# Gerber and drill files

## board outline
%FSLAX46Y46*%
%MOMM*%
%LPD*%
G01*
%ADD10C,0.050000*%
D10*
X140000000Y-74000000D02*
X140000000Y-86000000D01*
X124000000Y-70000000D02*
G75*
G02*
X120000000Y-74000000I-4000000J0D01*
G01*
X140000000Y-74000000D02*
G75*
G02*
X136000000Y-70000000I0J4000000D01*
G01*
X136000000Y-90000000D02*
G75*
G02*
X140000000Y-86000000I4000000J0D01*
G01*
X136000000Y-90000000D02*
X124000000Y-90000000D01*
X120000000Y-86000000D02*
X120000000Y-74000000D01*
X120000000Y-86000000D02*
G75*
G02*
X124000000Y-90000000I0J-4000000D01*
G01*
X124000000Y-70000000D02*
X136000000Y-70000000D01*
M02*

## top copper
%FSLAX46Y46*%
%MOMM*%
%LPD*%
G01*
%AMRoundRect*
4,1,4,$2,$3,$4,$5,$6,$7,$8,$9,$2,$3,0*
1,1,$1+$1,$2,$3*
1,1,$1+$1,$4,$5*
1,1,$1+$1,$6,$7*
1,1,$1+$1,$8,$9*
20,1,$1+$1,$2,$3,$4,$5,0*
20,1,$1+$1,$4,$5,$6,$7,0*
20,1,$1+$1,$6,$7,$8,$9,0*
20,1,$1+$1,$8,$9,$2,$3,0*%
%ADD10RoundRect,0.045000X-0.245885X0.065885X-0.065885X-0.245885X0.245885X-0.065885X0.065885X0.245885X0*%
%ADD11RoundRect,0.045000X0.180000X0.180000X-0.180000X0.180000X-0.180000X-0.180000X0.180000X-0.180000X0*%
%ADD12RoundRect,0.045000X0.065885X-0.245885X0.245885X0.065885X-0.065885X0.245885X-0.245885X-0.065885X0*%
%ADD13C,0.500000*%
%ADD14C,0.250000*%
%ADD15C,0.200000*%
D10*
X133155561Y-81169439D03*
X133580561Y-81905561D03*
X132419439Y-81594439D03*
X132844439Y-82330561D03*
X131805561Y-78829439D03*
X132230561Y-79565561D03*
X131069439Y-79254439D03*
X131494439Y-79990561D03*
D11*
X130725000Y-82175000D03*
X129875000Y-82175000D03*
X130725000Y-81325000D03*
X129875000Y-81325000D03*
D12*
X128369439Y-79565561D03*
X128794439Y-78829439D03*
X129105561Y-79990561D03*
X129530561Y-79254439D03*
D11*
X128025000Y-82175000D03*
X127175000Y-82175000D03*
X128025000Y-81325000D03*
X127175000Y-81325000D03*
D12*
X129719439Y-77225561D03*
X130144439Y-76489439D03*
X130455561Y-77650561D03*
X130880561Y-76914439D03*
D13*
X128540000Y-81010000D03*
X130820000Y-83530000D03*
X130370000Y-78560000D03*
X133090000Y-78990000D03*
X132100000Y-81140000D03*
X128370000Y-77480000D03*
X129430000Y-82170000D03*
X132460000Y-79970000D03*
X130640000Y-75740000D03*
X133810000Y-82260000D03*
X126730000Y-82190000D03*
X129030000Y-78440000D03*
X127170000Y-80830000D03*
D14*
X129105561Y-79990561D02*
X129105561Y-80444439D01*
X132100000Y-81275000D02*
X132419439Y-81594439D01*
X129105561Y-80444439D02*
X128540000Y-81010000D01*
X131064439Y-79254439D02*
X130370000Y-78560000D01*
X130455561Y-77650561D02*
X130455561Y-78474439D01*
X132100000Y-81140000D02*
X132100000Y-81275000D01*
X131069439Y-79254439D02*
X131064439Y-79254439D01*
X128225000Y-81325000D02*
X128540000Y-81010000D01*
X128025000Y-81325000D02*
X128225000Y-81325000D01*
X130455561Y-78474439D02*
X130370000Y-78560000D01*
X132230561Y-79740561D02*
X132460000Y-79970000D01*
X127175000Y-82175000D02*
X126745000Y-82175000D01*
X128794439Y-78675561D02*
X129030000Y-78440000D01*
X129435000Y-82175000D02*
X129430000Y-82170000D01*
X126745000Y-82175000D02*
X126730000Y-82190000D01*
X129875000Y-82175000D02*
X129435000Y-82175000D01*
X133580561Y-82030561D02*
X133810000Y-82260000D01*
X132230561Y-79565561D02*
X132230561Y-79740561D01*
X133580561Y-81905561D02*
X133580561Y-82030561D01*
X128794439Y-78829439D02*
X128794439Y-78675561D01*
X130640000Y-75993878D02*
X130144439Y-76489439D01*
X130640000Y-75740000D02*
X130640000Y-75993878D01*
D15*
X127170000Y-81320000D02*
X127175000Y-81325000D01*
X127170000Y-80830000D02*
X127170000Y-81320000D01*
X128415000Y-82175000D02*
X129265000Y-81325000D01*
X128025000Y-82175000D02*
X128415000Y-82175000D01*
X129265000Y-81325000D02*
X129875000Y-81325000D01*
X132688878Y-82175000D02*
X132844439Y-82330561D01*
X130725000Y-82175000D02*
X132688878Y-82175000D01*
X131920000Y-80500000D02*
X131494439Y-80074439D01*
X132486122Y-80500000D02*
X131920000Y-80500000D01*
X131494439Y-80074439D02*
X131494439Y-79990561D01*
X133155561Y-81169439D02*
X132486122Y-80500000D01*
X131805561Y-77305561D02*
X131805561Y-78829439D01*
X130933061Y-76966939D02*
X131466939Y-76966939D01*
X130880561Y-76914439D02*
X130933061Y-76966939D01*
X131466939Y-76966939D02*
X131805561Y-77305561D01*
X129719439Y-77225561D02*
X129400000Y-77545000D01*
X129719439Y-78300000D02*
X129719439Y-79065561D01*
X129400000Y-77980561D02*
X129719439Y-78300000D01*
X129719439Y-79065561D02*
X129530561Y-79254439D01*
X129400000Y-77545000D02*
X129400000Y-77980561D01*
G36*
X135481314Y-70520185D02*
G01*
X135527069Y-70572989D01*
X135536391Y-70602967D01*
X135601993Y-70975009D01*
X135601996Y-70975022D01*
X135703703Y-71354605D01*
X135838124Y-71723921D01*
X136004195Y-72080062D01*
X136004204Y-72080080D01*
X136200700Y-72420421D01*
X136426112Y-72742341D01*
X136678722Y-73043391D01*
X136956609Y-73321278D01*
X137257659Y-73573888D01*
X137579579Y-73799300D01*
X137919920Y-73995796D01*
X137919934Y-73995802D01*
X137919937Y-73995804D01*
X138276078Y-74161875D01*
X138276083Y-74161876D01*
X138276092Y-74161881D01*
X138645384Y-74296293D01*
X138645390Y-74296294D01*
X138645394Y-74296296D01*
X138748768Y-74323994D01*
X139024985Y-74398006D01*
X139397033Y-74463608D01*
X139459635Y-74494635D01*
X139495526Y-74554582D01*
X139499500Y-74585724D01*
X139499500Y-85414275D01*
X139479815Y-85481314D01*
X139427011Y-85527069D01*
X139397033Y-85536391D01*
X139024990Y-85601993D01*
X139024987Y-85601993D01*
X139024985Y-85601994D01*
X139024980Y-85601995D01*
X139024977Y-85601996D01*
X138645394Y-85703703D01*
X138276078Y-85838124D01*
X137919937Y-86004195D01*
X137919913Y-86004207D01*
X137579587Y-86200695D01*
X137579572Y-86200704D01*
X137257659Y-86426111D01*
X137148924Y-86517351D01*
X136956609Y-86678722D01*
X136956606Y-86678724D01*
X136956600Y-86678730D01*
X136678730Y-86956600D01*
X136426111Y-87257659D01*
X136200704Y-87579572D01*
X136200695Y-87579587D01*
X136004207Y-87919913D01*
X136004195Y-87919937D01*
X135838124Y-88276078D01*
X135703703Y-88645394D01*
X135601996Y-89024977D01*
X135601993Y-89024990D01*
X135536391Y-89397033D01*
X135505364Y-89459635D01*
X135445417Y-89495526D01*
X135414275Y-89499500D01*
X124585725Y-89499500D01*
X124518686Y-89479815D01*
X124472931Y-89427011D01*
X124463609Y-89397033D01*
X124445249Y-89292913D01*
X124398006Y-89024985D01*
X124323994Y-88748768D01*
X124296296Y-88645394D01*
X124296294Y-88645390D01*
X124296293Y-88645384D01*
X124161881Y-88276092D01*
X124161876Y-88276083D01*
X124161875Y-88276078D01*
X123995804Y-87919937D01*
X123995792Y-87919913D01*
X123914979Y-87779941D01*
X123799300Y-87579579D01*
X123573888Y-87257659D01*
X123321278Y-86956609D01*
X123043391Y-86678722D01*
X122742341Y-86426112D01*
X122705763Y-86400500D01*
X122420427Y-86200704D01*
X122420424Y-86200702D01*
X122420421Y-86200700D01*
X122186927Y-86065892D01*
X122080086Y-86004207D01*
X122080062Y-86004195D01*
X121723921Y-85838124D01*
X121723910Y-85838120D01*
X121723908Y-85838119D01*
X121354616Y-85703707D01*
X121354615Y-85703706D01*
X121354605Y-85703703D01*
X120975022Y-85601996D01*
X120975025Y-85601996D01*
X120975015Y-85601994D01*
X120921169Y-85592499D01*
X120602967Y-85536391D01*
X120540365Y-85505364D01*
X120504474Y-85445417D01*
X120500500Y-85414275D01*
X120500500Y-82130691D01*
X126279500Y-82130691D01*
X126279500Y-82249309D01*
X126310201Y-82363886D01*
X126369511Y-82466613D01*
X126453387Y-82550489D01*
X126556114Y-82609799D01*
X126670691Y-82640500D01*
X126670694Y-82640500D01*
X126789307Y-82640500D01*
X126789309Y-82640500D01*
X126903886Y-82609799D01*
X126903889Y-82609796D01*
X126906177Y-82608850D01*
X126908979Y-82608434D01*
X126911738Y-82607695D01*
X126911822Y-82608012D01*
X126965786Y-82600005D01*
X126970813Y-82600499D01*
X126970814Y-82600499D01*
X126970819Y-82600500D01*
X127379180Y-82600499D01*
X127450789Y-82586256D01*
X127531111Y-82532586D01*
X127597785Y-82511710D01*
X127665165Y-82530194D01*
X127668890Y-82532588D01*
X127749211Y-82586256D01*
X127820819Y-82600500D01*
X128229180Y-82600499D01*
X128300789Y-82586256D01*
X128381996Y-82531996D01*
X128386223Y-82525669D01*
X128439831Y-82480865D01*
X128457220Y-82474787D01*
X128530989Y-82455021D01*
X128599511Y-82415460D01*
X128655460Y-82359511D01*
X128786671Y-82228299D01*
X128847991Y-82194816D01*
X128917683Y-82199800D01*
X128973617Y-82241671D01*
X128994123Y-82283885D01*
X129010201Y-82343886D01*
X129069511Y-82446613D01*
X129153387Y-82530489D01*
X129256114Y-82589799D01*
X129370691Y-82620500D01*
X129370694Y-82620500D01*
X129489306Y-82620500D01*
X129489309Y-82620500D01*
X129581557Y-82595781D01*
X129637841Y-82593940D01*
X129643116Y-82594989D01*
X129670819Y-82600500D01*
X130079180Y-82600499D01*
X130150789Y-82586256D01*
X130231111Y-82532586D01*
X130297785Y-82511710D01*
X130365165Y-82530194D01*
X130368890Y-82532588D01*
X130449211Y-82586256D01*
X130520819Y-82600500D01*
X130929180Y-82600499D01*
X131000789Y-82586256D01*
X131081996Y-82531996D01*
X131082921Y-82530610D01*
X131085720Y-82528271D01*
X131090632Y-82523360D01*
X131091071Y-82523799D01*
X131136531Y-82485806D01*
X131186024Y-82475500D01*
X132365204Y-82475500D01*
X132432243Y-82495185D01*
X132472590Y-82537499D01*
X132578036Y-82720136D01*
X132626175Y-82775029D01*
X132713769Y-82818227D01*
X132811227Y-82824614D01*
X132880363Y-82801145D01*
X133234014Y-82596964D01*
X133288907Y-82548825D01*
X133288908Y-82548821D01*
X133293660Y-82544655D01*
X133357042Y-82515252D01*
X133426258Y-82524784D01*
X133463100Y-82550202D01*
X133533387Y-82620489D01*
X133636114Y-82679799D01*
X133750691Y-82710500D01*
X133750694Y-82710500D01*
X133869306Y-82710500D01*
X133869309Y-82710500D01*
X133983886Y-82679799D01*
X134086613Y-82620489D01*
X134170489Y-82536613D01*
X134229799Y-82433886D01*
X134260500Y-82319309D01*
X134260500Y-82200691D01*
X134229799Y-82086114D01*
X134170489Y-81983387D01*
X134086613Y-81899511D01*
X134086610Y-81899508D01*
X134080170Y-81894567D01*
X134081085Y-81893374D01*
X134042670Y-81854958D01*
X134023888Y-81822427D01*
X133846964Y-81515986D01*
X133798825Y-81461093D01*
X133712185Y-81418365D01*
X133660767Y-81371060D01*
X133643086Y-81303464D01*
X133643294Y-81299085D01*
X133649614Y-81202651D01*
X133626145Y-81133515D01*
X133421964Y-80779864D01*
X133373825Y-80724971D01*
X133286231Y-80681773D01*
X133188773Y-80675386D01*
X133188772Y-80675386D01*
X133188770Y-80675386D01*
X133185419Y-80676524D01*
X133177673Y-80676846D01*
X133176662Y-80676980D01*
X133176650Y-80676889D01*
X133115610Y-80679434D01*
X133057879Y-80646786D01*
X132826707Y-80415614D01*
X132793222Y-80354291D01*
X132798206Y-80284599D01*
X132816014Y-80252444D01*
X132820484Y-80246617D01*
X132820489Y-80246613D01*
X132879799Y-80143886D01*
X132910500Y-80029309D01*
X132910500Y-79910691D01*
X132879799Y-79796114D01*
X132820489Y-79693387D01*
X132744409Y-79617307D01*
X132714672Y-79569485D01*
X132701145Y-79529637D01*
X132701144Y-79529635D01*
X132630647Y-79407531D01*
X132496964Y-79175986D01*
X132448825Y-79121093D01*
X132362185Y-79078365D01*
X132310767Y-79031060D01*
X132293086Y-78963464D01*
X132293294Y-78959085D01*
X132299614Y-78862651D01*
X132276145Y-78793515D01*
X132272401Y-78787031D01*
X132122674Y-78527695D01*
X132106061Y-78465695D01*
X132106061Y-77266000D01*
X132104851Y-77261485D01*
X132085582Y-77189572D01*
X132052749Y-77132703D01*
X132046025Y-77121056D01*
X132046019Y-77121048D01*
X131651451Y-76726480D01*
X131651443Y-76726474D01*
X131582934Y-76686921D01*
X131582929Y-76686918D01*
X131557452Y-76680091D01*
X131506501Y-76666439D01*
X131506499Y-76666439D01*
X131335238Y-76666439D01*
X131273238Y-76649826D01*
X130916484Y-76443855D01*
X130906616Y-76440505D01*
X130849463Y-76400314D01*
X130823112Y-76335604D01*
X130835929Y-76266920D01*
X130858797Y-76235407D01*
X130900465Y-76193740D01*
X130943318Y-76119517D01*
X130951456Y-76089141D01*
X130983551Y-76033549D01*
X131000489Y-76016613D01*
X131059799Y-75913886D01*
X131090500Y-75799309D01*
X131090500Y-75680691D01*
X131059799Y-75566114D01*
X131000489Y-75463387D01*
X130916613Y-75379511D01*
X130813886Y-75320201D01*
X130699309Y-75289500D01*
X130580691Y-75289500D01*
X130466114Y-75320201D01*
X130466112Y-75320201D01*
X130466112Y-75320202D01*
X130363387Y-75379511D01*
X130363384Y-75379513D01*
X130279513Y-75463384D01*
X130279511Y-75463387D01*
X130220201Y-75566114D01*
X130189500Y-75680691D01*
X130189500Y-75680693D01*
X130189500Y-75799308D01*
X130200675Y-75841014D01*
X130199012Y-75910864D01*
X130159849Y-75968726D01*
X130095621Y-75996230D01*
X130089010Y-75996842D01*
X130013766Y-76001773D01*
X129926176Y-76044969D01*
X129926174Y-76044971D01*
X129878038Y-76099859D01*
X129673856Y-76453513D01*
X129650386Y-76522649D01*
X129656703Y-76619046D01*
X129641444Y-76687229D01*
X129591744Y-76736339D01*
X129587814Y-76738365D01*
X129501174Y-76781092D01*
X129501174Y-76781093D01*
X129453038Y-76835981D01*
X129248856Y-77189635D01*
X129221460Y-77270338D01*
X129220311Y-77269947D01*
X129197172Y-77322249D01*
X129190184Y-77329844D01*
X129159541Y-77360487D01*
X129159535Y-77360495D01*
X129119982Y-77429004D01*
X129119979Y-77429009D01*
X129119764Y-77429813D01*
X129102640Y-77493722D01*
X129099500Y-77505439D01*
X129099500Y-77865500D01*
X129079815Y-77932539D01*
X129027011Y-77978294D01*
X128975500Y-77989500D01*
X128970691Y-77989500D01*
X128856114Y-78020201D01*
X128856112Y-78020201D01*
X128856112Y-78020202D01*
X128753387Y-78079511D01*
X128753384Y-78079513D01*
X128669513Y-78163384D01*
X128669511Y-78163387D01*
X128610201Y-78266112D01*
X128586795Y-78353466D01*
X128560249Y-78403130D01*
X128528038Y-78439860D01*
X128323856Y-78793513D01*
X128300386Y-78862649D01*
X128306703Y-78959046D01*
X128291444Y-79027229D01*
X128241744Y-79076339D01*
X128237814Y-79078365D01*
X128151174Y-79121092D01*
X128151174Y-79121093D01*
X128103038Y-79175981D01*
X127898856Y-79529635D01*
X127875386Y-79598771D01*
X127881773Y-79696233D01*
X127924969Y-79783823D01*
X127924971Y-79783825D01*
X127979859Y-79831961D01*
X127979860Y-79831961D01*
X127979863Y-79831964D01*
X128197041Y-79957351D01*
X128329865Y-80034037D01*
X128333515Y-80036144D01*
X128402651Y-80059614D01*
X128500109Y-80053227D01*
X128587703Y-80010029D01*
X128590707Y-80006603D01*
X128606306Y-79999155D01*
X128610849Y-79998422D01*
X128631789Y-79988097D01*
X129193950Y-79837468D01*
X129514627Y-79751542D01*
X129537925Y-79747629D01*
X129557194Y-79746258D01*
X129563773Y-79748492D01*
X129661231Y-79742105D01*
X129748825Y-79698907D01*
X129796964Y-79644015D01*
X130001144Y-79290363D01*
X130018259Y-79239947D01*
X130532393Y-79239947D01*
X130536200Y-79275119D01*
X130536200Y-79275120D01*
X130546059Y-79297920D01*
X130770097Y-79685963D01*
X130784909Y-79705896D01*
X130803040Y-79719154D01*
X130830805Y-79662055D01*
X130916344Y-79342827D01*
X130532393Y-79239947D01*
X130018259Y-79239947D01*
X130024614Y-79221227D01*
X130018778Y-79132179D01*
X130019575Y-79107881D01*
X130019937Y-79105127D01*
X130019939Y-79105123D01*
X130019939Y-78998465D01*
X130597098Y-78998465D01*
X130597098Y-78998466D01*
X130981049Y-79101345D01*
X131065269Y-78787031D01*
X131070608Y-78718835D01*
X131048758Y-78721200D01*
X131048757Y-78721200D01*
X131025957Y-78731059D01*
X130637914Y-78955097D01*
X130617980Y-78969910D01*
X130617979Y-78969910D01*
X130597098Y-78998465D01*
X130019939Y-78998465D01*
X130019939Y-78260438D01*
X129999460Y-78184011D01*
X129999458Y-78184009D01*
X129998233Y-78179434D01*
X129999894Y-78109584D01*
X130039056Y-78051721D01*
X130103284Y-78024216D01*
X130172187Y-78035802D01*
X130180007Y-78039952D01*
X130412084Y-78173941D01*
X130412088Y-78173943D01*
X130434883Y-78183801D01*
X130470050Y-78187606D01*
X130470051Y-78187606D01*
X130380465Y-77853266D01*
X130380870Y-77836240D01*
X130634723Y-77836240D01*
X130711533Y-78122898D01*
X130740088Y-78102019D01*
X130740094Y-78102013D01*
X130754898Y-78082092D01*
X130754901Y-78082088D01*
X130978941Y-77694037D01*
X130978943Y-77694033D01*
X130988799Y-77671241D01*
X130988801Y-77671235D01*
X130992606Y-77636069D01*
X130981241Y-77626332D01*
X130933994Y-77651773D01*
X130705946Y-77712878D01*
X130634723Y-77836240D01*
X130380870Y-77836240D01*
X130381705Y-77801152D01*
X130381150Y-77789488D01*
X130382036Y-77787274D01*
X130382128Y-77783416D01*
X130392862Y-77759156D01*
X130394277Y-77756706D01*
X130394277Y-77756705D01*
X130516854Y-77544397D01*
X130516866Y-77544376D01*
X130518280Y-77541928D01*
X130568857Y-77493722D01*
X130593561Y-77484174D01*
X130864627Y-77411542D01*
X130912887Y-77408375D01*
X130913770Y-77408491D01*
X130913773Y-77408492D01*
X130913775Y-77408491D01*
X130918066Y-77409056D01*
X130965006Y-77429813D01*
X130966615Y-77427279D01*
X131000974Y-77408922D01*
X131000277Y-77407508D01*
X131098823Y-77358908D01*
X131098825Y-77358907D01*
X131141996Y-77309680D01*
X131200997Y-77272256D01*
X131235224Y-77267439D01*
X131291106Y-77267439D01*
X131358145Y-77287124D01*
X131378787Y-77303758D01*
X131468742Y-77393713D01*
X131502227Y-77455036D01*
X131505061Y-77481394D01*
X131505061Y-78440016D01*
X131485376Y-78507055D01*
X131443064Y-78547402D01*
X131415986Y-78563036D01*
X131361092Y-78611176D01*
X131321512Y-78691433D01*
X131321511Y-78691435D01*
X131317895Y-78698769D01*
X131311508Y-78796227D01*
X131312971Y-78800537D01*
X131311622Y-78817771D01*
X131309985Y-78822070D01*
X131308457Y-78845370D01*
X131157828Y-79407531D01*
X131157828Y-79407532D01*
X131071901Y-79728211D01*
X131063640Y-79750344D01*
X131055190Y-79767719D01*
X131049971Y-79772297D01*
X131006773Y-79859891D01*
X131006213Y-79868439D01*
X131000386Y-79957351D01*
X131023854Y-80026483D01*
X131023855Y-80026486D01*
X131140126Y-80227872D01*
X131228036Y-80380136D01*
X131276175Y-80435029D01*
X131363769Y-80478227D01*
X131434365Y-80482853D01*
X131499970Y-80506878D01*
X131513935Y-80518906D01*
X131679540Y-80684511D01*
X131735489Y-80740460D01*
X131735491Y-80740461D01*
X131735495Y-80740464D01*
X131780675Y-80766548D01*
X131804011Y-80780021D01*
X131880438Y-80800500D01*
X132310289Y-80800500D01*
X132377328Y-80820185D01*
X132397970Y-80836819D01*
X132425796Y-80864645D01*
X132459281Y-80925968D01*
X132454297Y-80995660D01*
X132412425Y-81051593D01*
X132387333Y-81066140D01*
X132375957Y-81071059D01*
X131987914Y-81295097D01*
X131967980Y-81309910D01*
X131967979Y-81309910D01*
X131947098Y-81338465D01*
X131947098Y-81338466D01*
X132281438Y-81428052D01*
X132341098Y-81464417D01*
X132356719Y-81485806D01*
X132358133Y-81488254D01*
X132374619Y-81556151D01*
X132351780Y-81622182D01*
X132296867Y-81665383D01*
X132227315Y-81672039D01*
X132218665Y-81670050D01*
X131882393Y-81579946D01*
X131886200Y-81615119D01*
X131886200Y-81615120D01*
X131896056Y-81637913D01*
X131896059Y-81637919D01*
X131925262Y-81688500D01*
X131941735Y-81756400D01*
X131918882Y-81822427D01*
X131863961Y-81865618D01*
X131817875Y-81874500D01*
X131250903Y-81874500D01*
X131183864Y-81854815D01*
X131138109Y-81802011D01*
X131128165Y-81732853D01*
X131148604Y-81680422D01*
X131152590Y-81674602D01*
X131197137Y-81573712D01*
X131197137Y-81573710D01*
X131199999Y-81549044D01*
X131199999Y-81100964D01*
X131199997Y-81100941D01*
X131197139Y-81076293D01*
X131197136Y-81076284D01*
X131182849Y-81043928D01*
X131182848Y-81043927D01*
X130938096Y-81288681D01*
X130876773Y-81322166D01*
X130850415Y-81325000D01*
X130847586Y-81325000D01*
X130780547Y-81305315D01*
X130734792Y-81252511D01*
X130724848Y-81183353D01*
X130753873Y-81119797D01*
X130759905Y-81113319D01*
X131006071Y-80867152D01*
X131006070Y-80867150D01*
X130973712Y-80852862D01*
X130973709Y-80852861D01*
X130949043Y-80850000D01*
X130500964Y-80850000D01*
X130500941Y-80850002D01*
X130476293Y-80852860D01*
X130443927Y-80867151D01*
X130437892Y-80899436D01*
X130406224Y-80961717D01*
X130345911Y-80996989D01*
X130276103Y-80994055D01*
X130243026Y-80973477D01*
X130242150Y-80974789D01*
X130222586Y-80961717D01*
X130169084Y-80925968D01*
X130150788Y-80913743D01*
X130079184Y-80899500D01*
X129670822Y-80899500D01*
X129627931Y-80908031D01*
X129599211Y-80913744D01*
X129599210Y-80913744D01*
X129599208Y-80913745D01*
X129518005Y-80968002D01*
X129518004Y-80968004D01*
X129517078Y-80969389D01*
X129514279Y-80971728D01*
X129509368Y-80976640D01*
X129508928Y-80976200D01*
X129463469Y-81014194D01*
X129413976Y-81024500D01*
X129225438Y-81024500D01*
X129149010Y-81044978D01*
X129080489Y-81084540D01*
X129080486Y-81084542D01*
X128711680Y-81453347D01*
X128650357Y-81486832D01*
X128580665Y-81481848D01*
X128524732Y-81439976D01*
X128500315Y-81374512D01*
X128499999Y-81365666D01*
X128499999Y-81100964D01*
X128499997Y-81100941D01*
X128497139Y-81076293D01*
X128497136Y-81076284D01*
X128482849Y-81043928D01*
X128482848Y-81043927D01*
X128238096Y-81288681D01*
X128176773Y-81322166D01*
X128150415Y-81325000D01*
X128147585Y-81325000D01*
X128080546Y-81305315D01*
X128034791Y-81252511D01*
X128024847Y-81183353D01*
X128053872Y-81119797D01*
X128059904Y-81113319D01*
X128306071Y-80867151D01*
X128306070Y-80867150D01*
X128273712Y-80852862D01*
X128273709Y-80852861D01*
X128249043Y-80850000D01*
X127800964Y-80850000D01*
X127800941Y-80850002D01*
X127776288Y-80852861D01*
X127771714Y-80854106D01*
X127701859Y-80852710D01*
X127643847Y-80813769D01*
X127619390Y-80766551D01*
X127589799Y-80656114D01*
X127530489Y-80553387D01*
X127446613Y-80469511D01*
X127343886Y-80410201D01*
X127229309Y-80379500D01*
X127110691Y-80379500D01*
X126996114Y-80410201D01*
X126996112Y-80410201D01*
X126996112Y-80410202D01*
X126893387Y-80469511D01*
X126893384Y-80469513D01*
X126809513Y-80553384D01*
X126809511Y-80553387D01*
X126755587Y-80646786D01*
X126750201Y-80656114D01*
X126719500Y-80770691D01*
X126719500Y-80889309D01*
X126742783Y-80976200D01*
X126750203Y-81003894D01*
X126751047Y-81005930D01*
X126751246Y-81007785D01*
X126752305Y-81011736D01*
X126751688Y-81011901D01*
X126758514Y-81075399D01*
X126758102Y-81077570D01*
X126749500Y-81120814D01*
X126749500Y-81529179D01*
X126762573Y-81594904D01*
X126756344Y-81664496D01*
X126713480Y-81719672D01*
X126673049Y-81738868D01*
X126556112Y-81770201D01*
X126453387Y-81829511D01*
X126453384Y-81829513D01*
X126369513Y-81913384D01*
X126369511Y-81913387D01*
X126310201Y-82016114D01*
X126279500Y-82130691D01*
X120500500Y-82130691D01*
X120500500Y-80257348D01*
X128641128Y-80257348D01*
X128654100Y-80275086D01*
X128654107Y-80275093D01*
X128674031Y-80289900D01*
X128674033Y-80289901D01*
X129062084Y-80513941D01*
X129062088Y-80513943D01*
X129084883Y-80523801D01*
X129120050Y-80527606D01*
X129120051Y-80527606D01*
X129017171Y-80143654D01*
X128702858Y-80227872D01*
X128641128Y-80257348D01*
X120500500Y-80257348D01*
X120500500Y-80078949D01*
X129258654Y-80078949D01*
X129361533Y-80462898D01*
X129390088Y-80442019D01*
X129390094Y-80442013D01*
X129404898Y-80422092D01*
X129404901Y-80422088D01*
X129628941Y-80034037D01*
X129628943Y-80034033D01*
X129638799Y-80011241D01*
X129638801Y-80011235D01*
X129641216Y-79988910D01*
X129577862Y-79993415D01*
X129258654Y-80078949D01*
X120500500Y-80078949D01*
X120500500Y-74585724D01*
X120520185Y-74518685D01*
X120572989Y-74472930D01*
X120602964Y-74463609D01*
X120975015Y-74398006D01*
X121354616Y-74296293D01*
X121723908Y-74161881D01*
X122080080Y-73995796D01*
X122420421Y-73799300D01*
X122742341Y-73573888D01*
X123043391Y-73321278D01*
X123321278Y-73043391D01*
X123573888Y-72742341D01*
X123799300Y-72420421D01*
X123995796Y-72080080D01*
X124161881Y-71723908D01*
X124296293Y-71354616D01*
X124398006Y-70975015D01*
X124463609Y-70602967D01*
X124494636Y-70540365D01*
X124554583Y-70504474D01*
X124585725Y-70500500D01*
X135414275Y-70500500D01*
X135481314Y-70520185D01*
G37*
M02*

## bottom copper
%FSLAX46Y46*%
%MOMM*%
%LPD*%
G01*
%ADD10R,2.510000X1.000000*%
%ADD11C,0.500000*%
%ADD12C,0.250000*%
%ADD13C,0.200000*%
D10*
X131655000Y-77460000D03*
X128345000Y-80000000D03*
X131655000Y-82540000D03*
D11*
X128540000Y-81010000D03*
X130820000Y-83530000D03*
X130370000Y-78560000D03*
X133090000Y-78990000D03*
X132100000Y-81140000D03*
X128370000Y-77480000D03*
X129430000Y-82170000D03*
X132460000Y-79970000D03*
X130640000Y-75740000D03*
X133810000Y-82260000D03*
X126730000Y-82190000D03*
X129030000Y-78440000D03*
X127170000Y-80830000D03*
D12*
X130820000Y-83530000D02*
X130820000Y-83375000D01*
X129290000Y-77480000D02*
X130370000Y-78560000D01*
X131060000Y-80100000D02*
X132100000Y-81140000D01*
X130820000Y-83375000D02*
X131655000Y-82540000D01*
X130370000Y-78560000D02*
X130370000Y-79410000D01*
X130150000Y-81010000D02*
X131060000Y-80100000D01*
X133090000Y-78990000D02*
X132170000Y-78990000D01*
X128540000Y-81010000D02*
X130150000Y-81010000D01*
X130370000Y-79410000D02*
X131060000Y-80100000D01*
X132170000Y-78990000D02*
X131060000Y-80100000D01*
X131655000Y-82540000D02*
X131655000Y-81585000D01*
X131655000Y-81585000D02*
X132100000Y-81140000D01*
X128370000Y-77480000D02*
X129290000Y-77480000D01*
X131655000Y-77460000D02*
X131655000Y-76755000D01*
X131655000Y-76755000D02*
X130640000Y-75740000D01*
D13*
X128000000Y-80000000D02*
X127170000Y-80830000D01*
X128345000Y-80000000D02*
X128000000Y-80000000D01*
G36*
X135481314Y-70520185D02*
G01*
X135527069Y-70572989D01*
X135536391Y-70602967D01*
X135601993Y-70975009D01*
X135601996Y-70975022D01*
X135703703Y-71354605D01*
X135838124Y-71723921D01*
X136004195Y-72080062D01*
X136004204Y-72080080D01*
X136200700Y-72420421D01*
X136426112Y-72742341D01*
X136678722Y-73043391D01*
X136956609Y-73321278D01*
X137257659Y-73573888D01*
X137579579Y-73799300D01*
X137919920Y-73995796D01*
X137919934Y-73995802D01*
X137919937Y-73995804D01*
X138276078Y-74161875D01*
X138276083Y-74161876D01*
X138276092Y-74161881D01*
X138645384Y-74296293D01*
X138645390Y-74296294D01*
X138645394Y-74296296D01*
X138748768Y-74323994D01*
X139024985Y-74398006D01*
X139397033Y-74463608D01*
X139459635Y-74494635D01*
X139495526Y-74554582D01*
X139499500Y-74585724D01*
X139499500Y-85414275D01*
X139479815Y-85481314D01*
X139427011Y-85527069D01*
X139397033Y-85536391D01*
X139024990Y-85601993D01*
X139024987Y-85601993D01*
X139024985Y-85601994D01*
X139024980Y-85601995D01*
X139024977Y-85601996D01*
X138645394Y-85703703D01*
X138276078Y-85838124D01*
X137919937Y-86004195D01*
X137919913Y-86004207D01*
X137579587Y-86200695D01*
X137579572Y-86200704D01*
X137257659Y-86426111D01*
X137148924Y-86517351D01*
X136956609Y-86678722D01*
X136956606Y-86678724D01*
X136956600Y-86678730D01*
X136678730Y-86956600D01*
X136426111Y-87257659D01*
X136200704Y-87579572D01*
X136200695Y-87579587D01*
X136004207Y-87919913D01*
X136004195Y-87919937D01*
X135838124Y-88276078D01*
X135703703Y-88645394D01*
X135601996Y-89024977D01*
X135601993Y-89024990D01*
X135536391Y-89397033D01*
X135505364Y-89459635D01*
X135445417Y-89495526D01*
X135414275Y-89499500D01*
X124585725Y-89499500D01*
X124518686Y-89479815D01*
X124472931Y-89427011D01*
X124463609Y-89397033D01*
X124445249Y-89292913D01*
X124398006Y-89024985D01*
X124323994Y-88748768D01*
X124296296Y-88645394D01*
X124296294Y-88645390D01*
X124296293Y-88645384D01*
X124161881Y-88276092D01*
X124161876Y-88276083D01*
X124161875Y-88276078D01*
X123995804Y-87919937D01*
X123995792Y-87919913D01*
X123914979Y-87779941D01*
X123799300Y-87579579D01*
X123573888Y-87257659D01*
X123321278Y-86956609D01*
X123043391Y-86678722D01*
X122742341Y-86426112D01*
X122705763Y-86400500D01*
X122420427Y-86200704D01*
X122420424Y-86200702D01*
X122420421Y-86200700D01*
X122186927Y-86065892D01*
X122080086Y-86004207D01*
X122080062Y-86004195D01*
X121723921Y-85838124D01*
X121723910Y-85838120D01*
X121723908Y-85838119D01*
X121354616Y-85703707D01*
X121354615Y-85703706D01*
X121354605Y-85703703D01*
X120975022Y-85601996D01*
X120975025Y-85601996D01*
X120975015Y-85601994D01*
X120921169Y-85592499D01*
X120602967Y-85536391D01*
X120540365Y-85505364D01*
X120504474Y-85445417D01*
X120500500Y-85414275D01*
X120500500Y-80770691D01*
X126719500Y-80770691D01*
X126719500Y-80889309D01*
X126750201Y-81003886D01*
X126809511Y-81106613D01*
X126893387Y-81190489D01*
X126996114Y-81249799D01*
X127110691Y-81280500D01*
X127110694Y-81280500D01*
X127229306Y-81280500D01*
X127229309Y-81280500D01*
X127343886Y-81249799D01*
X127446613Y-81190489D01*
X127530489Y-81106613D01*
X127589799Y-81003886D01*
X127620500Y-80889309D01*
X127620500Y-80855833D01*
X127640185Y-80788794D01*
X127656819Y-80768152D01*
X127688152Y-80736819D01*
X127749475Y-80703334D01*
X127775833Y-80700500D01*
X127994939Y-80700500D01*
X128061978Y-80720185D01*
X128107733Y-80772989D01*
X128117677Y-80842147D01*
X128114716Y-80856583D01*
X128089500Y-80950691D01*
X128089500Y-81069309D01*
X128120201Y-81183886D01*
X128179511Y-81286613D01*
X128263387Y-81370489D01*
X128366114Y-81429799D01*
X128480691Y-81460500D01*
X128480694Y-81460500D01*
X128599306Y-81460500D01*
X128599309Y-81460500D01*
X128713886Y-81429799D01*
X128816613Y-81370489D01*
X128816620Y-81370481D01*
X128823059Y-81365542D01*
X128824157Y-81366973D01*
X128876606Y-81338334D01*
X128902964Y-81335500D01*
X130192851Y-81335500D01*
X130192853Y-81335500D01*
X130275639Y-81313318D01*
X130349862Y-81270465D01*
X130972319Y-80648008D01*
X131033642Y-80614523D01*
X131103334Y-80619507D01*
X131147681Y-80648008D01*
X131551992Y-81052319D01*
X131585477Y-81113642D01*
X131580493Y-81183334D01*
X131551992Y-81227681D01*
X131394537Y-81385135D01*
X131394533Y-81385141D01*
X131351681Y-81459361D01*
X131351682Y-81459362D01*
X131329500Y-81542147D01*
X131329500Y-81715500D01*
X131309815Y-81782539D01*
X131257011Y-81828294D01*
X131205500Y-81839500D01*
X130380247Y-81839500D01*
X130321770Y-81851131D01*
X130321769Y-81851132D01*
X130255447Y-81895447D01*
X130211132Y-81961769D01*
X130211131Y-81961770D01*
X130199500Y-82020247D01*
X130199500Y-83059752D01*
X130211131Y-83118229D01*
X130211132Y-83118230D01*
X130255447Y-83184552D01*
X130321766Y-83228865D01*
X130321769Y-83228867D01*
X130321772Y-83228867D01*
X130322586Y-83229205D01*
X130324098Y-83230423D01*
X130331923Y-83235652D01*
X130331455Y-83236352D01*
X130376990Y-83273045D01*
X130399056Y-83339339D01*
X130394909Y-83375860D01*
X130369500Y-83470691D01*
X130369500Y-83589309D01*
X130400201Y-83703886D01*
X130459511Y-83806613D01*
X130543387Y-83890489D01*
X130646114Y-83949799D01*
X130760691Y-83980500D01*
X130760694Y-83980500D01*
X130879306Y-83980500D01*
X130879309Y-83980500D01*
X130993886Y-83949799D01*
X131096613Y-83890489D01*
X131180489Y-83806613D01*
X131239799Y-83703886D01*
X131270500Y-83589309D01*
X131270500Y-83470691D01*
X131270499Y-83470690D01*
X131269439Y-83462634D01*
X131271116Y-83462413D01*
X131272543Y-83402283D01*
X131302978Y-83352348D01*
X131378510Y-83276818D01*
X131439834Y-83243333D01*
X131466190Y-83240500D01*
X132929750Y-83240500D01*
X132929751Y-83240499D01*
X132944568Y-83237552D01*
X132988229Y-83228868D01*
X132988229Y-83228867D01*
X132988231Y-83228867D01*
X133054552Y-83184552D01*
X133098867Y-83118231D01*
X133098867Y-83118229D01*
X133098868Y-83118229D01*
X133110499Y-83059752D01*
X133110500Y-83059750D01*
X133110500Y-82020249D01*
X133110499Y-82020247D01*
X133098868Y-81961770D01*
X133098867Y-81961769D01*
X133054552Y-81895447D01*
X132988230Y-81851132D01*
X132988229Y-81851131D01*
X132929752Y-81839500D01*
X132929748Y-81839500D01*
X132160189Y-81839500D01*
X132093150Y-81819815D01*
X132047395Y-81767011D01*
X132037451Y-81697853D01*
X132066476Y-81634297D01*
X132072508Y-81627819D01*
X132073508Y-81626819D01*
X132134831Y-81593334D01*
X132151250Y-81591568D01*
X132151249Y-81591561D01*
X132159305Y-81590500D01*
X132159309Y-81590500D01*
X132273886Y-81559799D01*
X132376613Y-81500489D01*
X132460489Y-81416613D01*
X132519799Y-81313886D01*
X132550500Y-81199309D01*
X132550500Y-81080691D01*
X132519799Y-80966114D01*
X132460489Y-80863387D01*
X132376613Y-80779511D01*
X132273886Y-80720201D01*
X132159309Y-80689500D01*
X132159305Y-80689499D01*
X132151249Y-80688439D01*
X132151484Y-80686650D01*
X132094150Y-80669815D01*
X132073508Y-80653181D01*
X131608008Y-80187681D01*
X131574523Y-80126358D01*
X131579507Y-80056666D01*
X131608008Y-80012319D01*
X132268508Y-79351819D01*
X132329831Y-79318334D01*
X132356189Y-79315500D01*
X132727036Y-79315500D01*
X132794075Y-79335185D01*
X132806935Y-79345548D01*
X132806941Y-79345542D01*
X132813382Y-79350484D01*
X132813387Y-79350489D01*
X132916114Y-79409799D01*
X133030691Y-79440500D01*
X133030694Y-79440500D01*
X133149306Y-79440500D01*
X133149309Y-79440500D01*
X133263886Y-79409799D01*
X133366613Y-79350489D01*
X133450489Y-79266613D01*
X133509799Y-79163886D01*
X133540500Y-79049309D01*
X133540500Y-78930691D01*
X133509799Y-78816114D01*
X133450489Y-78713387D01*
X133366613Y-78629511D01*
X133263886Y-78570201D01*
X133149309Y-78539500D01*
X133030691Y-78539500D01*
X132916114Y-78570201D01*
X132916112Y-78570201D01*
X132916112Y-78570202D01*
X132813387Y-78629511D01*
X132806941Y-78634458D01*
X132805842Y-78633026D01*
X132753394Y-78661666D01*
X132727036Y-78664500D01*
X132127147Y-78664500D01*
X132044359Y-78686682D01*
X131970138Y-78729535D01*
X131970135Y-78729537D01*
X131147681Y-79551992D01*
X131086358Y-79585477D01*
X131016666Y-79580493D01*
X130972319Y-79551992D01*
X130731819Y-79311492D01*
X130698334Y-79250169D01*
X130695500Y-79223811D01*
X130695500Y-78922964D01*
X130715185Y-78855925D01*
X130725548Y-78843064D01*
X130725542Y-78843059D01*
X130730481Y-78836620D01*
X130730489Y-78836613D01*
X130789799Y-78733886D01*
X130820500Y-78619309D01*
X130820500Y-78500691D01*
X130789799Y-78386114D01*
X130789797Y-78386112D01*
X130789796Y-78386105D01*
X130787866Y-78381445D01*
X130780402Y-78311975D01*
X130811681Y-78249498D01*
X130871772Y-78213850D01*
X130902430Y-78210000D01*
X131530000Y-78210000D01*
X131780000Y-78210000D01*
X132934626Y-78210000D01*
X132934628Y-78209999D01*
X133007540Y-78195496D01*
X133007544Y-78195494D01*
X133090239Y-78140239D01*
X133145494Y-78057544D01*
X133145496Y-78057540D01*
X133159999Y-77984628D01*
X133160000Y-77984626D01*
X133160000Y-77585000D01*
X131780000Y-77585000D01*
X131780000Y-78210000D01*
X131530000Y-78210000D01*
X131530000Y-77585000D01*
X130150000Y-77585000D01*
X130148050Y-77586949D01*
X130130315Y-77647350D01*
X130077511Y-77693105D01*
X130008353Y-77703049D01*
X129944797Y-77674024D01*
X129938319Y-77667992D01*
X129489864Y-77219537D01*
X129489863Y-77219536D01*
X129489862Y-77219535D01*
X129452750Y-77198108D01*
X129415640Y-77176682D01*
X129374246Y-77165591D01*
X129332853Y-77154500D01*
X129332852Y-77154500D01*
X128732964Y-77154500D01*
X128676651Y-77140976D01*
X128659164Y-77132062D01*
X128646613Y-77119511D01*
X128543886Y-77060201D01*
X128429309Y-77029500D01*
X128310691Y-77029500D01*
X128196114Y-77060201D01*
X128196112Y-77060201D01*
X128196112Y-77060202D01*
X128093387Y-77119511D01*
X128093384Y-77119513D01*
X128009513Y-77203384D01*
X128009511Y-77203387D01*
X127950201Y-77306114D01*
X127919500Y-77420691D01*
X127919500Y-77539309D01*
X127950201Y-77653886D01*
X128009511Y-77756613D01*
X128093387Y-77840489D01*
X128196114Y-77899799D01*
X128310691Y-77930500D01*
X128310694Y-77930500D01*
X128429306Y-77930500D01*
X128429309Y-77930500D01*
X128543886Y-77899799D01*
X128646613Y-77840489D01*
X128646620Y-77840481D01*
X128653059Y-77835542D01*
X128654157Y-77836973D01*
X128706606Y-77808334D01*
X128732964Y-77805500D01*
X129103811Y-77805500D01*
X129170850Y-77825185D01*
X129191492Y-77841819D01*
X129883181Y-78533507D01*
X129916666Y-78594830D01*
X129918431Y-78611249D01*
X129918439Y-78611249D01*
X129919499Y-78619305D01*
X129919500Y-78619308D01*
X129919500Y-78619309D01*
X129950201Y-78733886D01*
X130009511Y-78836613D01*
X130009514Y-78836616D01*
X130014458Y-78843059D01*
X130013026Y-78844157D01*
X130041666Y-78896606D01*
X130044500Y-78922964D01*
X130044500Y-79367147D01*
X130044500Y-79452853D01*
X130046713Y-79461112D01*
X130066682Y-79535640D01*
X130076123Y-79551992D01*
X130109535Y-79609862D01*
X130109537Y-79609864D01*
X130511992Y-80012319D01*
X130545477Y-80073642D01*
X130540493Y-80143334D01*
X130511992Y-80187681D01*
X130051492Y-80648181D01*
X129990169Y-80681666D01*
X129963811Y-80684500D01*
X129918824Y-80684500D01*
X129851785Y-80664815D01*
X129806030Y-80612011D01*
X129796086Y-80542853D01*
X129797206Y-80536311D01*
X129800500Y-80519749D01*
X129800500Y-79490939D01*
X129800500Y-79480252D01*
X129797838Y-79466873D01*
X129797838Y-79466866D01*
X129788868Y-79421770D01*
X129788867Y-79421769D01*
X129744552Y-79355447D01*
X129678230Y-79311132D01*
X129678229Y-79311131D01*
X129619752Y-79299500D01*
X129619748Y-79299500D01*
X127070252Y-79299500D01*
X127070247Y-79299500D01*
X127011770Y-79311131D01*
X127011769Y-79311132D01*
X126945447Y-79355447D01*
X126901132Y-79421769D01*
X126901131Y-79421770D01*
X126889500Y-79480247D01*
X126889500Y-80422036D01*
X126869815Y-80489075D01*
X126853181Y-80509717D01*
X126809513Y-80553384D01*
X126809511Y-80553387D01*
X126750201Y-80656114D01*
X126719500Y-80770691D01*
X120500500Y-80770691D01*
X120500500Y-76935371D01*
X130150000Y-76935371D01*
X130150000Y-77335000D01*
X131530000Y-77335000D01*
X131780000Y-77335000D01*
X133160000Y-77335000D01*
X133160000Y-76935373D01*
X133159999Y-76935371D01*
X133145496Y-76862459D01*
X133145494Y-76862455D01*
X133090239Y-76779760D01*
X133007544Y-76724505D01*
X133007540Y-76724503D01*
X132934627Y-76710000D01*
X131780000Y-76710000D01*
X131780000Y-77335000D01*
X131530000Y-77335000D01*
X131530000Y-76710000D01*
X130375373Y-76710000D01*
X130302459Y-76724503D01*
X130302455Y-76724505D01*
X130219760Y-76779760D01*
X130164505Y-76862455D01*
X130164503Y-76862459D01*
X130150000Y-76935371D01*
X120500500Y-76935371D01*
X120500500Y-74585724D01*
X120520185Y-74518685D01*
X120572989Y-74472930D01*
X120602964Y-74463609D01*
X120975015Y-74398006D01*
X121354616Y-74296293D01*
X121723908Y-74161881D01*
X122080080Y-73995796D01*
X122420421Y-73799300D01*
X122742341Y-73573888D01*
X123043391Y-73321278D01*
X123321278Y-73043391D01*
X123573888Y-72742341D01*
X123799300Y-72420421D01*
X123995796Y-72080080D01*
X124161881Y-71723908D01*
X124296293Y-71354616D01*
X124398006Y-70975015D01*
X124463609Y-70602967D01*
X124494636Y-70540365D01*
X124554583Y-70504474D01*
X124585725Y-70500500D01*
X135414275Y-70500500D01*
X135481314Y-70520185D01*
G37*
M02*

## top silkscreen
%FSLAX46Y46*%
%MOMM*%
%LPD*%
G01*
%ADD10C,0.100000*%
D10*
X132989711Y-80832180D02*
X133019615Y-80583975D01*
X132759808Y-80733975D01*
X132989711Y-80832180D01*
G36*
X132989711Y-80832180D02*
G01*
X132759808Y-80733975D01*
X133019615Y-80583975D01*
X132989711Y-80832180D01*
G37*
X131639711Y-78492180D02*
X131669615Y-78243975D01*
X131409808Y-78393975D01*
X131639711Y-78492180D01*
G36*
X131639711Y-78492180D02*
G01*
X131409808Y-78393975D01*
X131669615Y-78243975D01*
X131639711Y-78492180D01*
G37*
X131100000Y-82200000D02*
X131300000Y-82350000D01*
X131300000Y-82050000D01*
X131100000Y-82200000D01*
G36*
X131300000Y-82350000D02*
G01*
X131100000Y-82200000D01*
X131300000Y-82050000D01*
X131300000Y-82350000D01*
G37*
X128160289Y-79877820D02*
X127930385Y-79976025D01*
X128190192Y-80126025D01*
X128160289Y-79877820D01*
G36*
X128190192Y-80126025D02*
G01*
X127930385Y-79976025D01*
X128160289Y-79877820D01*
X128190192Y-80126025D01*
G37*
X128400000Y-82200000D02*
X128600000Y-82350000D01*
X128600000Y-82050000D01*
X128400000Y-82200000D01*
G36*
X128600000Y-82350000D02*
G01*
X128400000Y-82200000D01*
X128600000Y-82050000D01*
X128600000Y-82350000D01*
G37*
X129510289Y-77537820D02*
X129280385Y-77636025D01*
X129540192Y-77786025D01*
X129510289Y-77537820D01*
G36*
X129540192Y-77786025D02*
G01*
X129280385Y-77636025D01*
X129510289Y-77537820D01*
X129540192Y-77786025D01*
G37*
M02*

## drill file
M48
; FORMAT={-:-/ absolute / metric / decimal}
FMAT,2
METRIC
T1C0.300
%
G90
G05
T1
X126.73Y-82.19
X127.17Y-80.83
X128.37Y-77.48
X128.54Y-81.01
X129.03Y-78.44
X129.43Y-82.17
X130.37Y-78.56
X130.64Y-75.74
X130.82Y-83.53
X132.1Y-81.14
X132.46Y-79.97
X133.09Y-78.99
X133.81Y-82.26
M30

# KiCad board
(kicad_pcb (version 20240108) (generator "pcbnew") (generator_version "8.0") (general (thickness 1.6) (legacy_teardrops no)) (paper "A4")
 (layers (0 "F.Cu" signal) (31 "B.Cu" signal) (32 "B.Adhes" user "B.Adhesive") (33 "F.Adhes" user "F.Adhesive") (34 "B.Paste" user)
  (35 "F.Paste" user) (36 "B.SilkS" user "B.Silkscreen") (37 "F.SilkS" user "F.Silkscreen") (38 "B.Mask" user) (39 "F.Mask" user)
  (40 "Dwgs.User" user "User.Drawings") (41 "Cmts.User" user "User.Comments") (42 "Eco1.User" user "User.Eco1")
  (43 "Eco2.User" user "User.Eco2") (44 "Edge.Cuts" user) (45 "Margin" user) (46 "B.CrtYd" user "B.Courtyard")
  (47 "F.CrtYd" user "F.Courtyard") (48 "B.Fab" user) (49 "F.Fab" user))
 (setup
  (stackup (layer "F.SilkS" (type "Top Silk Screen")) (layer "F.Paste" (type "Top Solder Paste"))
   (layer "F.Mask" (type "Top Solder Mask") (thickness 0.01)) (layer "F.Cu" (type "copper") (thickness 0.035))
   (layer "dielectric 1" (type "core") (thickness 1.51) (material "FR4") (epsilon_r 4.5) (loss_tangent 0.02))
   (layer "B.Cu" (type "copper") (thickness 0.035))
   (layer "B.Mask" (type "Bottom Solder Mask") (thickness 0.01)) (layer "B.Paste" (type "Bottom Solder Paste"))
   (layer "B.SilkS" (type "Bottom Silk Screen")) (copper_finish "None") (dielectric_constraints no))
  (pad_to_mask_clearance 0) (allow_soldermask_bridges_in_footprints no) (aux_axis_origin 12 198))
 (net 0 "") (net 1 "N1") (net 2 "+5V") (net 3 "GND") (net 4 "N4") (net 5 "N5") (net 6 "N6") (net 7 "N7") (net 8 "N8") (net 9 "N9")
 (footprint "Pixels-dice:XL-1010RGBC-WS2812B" (layer "F.Cu") (at 133 81.75 -60)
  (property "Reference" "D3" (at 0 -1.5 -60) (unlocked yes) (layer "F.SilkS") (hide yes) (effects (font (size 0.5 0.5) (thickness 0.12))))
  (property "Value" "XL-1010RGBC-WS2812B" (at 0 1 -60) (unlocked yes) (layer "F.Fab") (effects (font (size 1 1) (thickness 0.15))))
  (fp_poly (pts (xy -0.8 -0.449999) (xy -1 -0.6) (xy -0.999999 -0.3)) (stroke (width 0.1) (type solid)) (fill solid) (layer "F.SilkS"))
  (pad "1" smd roundrect (at -0.425 -0.425 300) (size 0.45 0.45) (layers "F.Cu" "F.Paste" "F.Mask") (roundrect_rratio 0.1) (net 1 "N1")
   (thermal_bridge_angle 45))
  (pad "2" smd roundrect (at 0.425 -0.425 300) (size 0.45 0.45) (layers "F.Cu" "F.Paste" "F.Mask") (roundrect_rratio 0.1) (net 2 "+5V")
   (thermal_bridge_angle 45))
  (pad "3" smd roundrect (at -0.425 0.425 300) (size 0.45 0.45) (layers "F.Cu" "F.Paste" "F.Mask") (roundrect_rratio 0.1) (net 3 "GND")
   (thermal_bridge_angle 45))
  (pad "4" smd roundrect (at 0.425 0.425 300) (size 0.45 0.45) (layers "F.Cu" "F.Paste" "F.Mask") (roundrect_rratio 0.1) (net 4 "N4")
   (thermal_bridge_angle 45)))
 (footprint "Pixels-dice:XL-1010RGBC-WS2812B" (layer "F.Cu") (at 131.65 79.41 -60)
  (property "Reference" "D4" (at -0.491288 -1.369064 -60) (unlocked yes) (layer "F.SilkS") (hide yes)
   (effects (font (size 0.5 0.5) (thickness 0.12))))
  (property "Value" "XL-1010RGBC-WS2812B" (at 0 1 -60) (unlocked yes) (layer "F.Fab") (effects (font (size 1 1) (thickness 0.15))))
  (fp_poly (pts (xy -0.8 -0.449999) (xy -1 -0.6) (xy -0.999999 -0.3)) (stroke (width 0.1) (type solid)) (fill solid) (layer "F.SilkS"))
  (pad "1" smd roundrect (at -0.425 -0.425 300) (size 0.45 0.45) (layers "F.Cu" "F.Paste" "F.Mask") (roundrect_rratio 0.1) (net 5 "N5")
   (thermal_bridge_angle 45))
  (pad "2" smd roundrect (at 0.425 -0.425 300) (size 0.45 0.45) (layers "F.Cu" "F.Paste" "F.Mask") (roundrect_rratio 0.1) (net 2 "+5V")
   (thermal_bridge_angle 45))
  (pad "3" smd roundrect (at -0.425 0.425 300) (size 0.45 0.45) (layers "F.Cu" "F.Paste" "F.Mask") (roundrect_rratio 0.1) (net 3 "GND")
   (thermal_bridge_angle 45))
  (pad "4" smd roundrect (at 0.425 0.425 300) (size 0.45 0.45) (layers "F.Cu" "F.Paste" "F.Mask") (roundrect_rratio 0.1) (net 1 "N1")
   (thermal_bridge_angle 45)))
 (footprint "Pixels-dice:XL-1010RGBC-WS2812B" (layer "F.Cu") (at 130.3 81.75 180)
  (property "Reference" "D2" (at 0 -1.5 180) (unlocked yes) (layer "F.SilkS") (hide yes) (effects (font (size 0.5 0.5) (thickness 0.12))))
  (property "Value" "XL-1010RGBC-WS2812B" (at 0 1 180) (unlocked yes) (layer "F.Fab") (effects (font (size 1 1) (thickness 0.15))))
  (fp_poly (pts (xy -0.8 -0.45) (xy -1 -0.6) (xy -1 -0.3)) (stroke (width 0.1) (type solid)) (fill solid) (layer "F.SilkS"))
  (pad "1" smd roundrect (at -0.425 -0.425 180) (size 0.45 0.45) (layers "F.Cu" "F.Paste" "F.Mask") (roundrect_rratio 0.1) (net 4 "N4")
   (thermal_bridge_angle 45))
  (pad "2" smd roundrect (at 0.425 -0.425 180) (size 0.45 0.45) (layers "F.Cu" "F.Paste" "F.Mask") (roundrect_rratio 0.1) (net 2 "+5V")
   (thermal_bridge_angle 45))
  (pad "3" smd roundrect (at -0.425 0.425 180) (size 0.45 0.45) (layers "F.Cu" "F.Paste" "F.Mask") (roundrect_rratio 0.1) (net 3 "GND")
   (thermal_bridge_angle 45))
  (pad "4" smd roundrect (at 0.425 0.425 180) (size 0.45 0.45) (layers "F.Cu" "F.Paste" "F.Mask") (roundrect_rratio 0.1) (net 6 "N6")
   (thermal_bridge_angle 45)))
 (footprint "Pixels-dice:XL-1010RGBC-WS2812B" (layer "F.Cu") (at 128.95 79.41 60)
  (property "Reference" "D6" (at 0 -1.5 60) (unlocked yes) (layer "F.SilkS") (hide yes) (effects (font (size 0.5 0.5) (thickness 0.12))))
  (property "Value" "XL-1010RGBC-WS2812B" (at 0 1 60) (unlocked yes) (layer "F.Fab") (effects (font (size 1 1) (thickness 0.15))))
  (fp_poly (pts (xy -0.8 -0.45) (xy -1 -0.6) (xy -1 -0.300001)) (stroke (width 0.1) (type solid)) (fill solid) (layer "F.SilkS"))
  (pad "1" smd roundrect (at -0.425 -0.425 60) (size 0.45 0.45) (layers "F.Cu" "F.Paste" "F.Mask") (roundrect_rratio 0.1) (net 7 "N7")
   (thermal_bridge_angle 45))
  (pad "2" smd roundrect (at 0.425 -0.425 60) (size 0.45 0.45) (layers "F.Cu" "F.Paste" "F.Mask") (roundrect_rratio 0.1) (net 2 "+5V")
   (thermal_bridge_angle 45))
  (pad "3" smd roundrect (at -0.425 0.425 60) (size 0.45 0.45) (layers "F.Cu" "F.Paste" "F.Mask") (roundrect_rratio 0.1) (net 3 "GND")
   (thermal_bridge_angle 45))
  (pad "4" smd roundrect (at 0.425 0.425 60) (size 0.45 0.45) (layers "F.Cu" "F.Paste" "F.Mask") (roundrect_rratio 0.1) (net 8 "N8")
   (thermal_bridge_angle 45)))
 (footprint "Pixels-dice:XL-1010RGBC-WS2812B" (layer "F.Cu") (at 127.6 81.75 180)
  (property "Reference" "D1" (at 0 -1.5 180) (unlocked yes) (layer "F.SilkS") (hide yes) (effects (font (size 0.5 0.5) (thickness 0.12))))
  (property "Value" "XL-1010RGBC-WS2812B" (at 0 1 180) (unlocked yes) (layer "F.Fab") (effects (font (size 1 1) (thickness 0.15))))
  (fp_poly (pts (xy -0.8 -0.45) (xy -1 -0.6) (xy -1 -0.3)) (stroke (width 0.1) (type solid)) (fill solid) (layer "F.SilkS"))
  (pad "1" smd roundrect (at -0.425 -0.425 180) (size 0.45 0.45) (layers "F.Cu" "F.Paste" "F.Mask") (roundrect_rratio 0.1) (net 6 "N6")
   (thermal_bridge_angle 45))
  (pad "2" smd roundrect (at 0.425 -0.425 180) (size 0.45 0.45) (layers "F.Cu" "F.Paste" "F.Mask") (roundrect_rratio 0.1) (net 2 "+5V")
   (thermal_bridge_angle 45))
  (pad "3" smd roundrect (at -0.425 0.425 180) (size 0.45 0.45) (layers "F.Cu" "F.Paste" "F.Mask") (roundrect_rratio 0.1) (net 3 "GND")
   (thermal_bridge_angle 45))
  (pad "4" smd roundrect (at 0.425 0.425 180) (size 0.45 0.45) (layers "F.Cu" "F.Paste" "F.Mask") (roundrect_rratio 0.1) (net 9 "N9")
   (thermal_bridge_angle 45)))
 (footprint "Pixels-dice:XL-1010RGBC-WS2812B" (layer "F.Cu") (at 130.3 77.07 60)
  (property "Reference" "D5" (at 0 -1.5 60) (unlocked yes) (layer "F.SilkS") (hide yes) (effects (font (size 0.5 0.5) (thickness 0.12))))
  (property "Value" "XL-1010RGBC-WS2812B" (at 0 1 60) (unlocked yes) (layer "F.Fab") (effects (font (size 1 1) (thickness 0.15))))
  (fp_poly (pts (xy -0.8 -0.45) (xy -1 -0.6) (xy -1 -0.300001)) (stroke (width 0.1) (type solid)) (fill solid) (layer "F.SilkS"))
  (pad "1" smd roundrect (at -0.425 -0.425 60) (size 0.45 0.45) (layers "F.Cu" "F.Paste" "F.Mask") (roundrect_rratio 0.1) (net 8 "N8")
   (thermal_bridge_angle 45))
  (pad "2" smd roundrect (at 0.425 -0.425 60) (size 0.45 0.45) (layers "F.Cu" "F.Paste" "F.Mask") (roundrect_rratio 0.1) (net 2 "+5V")
   (thermal_bridge_angle 45))
  (pad "3" smd roundrect (at -0.425 0.425 60) (size 0.45 0.45) (layers "F.Cu" "F.Paste" "F.Mask") (roundrect_rratio 0.1) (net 3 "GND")
   (thermal_bridge_angle 45))
  (pad "4" smd roundrect (at 0.425 0.425 60) (size 0.45 0.45) (layers "F.Cu" "F.Paste" "F.Mask") (roundrect_rratio 0.1) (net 5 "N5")
   (thermal_bridge_angle 45)))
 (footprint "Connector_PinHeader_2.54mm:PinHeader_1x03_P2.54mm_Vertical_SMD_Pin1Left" (layer "B.Cu") (at 130 80 180)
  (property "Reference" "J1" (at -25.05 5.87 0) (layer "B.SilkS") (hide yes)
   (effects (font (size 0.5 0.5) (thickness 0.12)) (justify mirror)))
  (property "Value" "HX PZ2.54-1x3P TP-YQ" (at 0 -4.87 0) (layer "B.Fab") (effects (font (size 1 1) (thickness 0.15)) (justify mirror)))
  (pad "1" smd rect (at -1.655 2.54 180) (size 2.51 1) (layers "B.Cu" "B.Paste" "B.Mask") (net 2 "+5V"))
  (pad "2" smd rect (at 1.655 0 180) (size 2.51 1) (layers "B.Cu" "B.Paste" "B.Mask") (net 9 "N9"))
  (pad "3" smd rect (at -1.655 -2.54 180) (size 2.51 1) (layers "B.Cu" "B.Paste" "B.Mask") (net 3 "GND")))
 (gr_line (start 140 74) (end 140 86) (stroke (width 0.05) (type default)) (layer "Edge.Cuts"))
 (gr_arc (start 124 70) (mid 122.828427 72.828427) (end 120 74) (stroke (width 0.05) (type default)) (layer "Edge.Cuts"))
 (gr_arc (start 140 74) (mid 137.171573 72.828427) (end 136 70) (stroke (width 0.05) (type default)) (layer "Edge.Cuts"))
 (gr_arc (start 136 90) (mid 137.171573 87.171573) (end 140 86) (stroke (width 0.05) (type default)) (layer "Edge.Cuts"))
 (gr_line (start 136 90) (end 124 90) (stroke (width 0.05) (type default)) (layer "Edge.Cuts"))
 (gr_line (start 120 86) (end 120 74) (stroke (width 0.05) (type default)) (layer "Edge.Cuts"))
 (gr_arc (start 120 86) (mid 122.828427 87.171573) (end 124 90) (stroke (width 0.05) (type default)) (layer "Edge.Cuts"))
 (gr_line (start 124 70) (end 136 70) (stroke (width 0.05) (type default)) (layer "Edge.Cuts"))
 (segment (start 129.105561 79.990561) (end 129.105561 80.444439) (width 0.25) (layer "F.Cu") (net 3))
 (segment (start 132.1 81.275) (end 132.419439 81.594439) (width 0.25) (layer "F.Cu") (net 3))
 (segment (start 129.105561 80.444439) (end 128.54 81.01) (width 0.25) (layer "F.Cu") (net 3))
 (segment (start 131.064439 79.254439) (end 130.37 78.56) (width 0.25) (layer "F.Cu") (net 3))
 (segment (start 130.455561 77.650561) (end 130.455561 78.474439) (width 0.25) (layer "F.Cu") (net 3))
 (segment (start 132.1 81.14) (end 132.1 81.275) (width 0.25) (layer "F.Cu") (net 3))
 (segment (start 131.069439 79.254439) (end 131.064439 79.254439) (width 0.25) (layer "F.Cu") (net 3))
 (segment (start 128.225 81.325) (end 128.54 81.01) (width 0.25) (layer "F.Cu") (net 3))
 (segment (start 128.025 81.325) (end 128.225 81.325) (width 0.25) (layer "F.Cu") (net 3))
 (segment (start 130.455561 78.474439) (end 130.37 78.56) (width 0.25) (layer "F.Cu") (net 3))
 (via (at 128.54 81.01) (size 0.5) (drill 0.3) (layers "F.Cu" "B.Cu") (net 3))
 (via (at 130.82 83.53) (size 0.5) (drill 0.3) (layers "F.Cu" "B.Cu") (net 3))
 (via (at 130.37 78.56) (size 0.5) (drill 0.3) (layers "F.Cu" "B.Cu") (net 3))
 (via (at 133.09 78.99) (size 0.5) (drill 0.3) (layers "F.Cu" "B.Cu") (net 3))
 (via (at 132.1 81.14) (size 0.5) (drill 0.3) (layers "F.Cu" "B.Cu") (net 3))
 (via (at 128.37 77.48) (size 0.5) (drill 0.3) (layers "F.Cu" "B.Cu") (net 3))
 (segment (start 130.82 83.53) (end 130.82 83.375) (width 0.25) (layer "B.Cu") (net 3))
 (segment (start 129.29 77.48) (end 130.37 78.56) (width 0.25) (layer "B.Cu") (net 3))
 (segment (start 131.06 80.1) (end 132.1 81.14) (width 0.25) (layer "B.Cu") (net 3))
 (segment (start 130.82 83.375) (end 131.655 82.54) (width 0.25) (layer "B.Cu") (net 3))
 (segment (start 130.37 78.56) (end 130.37 79.41) (width 0.25) (layer "B.Cu") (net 3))
 (segment (start 130.15 81.01) (end 131.06 80.1) (width 0.25) (layer "B.Cu") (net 3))
 (segment (start 133.09 78.99) (end 132.17 78.99) (width 0.25) (layer "B.Cu") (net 3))
 (segment (start 128.54 81.01) (end 130.15 81.01) (width 0.25) (layer "B.Cu") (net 3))
 (segment (start 130.37 79.41) (end 131.06 80.1) (width 0.25) (layer "B.Cu") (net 3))
 (segment (start 132.17 78.99) (end 131.06 80.1) (width 0.25) (layer "B.Cu") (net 3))
 (segment (start 131.655 82.54) (end 131.655 81.585) (width 0.25) (layer "B.Cu") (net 3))
 (segment (start 131.655 81.585) (end 132.1 81.14) (width 0.25) (layer "B.Cu") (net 3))
 (segment (start 128.37 77.48) (end 129.29 77.48) (width 0.25) (layer "B.Cu") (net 3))
 (segment (start 132.230561 79.740561) (end 132.46 79.97) (width 0.25) (layer "F.Cu") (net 2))
 (segment (start 127.175 82.175) (end 126.745 82.175) (width 0.25) (layer "F.Cu") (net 2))
 (segment (start 128.794439 78.675561) (end 129.03 78.44) (width 0.25) (layer "F.Cu") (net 2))
 (segment (start 129.435 82.175) (end 129.43 82.17) (width 0.25) (layer "F.Cu") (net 2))
 (segment (start 126.745 82.175) (end 126.73 82.19) (width 0.25) (layer "F.Cu") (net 2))
 (segment (start 129.875 82.175) (end 129.435 82.175) (width 0.25) (layer "F.Cu") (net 2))
 (segment (start 133.580561 82.030561) (end 133.81 82.26) (width 0.25) (layer "F.Cu") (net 2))
 (segment (start 132.230561 79.565561) (end 132.230561 79.740561) (width 0.25) (layer "F.Cu") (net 2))
 (segment (start 133.580561 81.905561) (end 133.580561 82.030561) (width 0.25) (layer "F.Cu") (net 2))
 (segment (start 128.794439 78.829439) (end 128.794439 78.675561) (width 0.25) (layer "F.Cu") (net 2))
 (segment (start 130.64 75.993878) (end 130.144439 76.489439) (width 0.25) (layer "F.Cu") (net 2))
 (segment (start 130.64 75.74) (end 130.64 75.993878) (width 0.25) (layer "F.Cu") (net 2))
 (via (at 129.43 82.17) (size 0.5) (drill 0.3) (layers "F.Cu" "B.Cu") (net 2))
 (via (at 132.46 79.97) (size 0.5) (drill 0.3) (layers "F.Cu" "B.Cu") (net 2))
 (via (at 130.64 75.74) (size 0.5) (drill 0.3) (layers "F.Cu" "B.Cu") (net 2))
 (via (at 133.81 82.26) (size 0.5) (drill 0.3) (layers "F.Cu" "B.Cu") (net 2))
 (via (at 126.73 82.19) (size 0.5) (drill 0.3) (layers "F.Cu" "B.Cu") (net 2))
 (via (at 129.03 78.44) (size 0.5) (drill 0.3) (layers "F.Cu" "B.Cu") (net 2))
 (segment (start 131.655 77.46) (end 131.655 76.755) (width 0.25) (layer "B.Cu") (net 2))
 (segment (start 131.655 76.755) (end 130.64 75.74) (width 0.25) (layer "B.Cu") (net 2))
 (segment (start 127.17 81.32) (end 127.175 81.325) (width 0.2) (layer "F.Cu") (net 9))
 (segment (start 127.17 80.83) (end 127.17 81.32) (width 0.2) (layer "F.Cu") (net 9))
 (via (at 127.17 80.83) (size 0.5) (drill 0.3) (layers "F.Cu" "B.Cu") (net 9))
 (segment (start 128 80) (end 127.17 80.83) (width 0.2) (layer "B.Cu") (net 9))
 (segment (start 128.345 80) (end 128 80) (width 0.2) (layer "B.Cu") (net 9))
 (segment (start 128.415 82.175) (end 129.265 81.325) (width 0.2) (layer "F.Cu") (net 6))
 (segment (start 128.025 82.175) (end 128.415 82.175) (width 0.2) (layer "F.Cu") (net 6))
 (segment (start 129.265 81.325) (end 129.875 81.325) (width 0.2) (layer "F.Cu") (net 6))
 (segment (start 132.688878 82.175) (end 132.844439 82.330561) (width 0.2) (layer "F.Cu") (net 4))
 (segment (start 130.725 82.175) (end 132.688878 82.175) (width 0.2) (layer "F.Cu") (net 4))
 (segment (start 131.92 80.5) (end 131.494439 80.074439) (width 0.2) (layer "F.Cu") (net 1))
 (segment (start 132.486122 80.5) (end 131.92 80.5) (width 0.2) (layer "F.Cu") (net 1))
 (segment (start 131.494439 80.074439) (end 131.494439 79.990561) (width 0.2) (layer "F.Cu") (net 1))
 (segment (start 133.155561 81.169439) (end 132.486122 80.5) (width 0.2) (layer "F.Cu") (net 1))
 (segment (start 131.805561 77.305561) (end 131.805561 78.829439) (width 0.2) (layer "F.Cu") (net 5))
 (segment (start 130.933061 76.966939) (end 131.466939 76.966939) (width 0.2) (layer "F.Cu") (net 5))
 (segment (start 130.880561 76.914439) (end 130.933061 76.966939) (width 0.2) (layer "F.Cu") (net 5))
 (segment (start 131.466939 76.966939) (end 131.805561 77.305561) (width 0.2) (layer "F.Cu") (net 5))
 (segment (start 129.719439 77.225561) (end 129.4 77.545) (width 0.2) (layer "F.Cu") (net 8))
 (segment (start 129.719439 78.3) (end 129.719439 79.065561) (width 0.2) (layer "F.Cu") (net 8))
 (segment (start 129.4 77.980561) (end 129.719439 78.3) (width 0.2) (layer "F.Cu") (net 8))
 (segment (start 129.719439 79.065561) (end 129.530561 79.254439) (width 0.2) (layer "F.Cu") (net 8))
 (segment (start 129.4 77.545) (end 129.4 77.980561) (width 0.2) (layer "F.Cu") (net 8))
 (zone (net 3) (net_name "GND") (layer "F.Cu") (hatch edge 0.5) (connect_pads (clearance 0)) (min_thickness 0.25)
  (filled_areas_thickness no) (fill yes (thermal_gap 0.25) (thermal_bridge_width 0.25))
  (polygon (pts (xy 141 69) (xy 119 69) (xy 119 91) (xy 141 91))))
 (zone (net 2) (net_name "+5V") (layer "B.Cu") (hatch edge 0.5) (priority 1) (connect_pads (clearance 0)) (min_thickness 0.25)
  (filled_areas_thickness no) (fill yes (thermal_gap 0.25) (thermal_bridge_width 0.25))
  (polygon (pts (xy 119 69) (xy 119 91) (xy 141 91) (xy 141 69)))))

